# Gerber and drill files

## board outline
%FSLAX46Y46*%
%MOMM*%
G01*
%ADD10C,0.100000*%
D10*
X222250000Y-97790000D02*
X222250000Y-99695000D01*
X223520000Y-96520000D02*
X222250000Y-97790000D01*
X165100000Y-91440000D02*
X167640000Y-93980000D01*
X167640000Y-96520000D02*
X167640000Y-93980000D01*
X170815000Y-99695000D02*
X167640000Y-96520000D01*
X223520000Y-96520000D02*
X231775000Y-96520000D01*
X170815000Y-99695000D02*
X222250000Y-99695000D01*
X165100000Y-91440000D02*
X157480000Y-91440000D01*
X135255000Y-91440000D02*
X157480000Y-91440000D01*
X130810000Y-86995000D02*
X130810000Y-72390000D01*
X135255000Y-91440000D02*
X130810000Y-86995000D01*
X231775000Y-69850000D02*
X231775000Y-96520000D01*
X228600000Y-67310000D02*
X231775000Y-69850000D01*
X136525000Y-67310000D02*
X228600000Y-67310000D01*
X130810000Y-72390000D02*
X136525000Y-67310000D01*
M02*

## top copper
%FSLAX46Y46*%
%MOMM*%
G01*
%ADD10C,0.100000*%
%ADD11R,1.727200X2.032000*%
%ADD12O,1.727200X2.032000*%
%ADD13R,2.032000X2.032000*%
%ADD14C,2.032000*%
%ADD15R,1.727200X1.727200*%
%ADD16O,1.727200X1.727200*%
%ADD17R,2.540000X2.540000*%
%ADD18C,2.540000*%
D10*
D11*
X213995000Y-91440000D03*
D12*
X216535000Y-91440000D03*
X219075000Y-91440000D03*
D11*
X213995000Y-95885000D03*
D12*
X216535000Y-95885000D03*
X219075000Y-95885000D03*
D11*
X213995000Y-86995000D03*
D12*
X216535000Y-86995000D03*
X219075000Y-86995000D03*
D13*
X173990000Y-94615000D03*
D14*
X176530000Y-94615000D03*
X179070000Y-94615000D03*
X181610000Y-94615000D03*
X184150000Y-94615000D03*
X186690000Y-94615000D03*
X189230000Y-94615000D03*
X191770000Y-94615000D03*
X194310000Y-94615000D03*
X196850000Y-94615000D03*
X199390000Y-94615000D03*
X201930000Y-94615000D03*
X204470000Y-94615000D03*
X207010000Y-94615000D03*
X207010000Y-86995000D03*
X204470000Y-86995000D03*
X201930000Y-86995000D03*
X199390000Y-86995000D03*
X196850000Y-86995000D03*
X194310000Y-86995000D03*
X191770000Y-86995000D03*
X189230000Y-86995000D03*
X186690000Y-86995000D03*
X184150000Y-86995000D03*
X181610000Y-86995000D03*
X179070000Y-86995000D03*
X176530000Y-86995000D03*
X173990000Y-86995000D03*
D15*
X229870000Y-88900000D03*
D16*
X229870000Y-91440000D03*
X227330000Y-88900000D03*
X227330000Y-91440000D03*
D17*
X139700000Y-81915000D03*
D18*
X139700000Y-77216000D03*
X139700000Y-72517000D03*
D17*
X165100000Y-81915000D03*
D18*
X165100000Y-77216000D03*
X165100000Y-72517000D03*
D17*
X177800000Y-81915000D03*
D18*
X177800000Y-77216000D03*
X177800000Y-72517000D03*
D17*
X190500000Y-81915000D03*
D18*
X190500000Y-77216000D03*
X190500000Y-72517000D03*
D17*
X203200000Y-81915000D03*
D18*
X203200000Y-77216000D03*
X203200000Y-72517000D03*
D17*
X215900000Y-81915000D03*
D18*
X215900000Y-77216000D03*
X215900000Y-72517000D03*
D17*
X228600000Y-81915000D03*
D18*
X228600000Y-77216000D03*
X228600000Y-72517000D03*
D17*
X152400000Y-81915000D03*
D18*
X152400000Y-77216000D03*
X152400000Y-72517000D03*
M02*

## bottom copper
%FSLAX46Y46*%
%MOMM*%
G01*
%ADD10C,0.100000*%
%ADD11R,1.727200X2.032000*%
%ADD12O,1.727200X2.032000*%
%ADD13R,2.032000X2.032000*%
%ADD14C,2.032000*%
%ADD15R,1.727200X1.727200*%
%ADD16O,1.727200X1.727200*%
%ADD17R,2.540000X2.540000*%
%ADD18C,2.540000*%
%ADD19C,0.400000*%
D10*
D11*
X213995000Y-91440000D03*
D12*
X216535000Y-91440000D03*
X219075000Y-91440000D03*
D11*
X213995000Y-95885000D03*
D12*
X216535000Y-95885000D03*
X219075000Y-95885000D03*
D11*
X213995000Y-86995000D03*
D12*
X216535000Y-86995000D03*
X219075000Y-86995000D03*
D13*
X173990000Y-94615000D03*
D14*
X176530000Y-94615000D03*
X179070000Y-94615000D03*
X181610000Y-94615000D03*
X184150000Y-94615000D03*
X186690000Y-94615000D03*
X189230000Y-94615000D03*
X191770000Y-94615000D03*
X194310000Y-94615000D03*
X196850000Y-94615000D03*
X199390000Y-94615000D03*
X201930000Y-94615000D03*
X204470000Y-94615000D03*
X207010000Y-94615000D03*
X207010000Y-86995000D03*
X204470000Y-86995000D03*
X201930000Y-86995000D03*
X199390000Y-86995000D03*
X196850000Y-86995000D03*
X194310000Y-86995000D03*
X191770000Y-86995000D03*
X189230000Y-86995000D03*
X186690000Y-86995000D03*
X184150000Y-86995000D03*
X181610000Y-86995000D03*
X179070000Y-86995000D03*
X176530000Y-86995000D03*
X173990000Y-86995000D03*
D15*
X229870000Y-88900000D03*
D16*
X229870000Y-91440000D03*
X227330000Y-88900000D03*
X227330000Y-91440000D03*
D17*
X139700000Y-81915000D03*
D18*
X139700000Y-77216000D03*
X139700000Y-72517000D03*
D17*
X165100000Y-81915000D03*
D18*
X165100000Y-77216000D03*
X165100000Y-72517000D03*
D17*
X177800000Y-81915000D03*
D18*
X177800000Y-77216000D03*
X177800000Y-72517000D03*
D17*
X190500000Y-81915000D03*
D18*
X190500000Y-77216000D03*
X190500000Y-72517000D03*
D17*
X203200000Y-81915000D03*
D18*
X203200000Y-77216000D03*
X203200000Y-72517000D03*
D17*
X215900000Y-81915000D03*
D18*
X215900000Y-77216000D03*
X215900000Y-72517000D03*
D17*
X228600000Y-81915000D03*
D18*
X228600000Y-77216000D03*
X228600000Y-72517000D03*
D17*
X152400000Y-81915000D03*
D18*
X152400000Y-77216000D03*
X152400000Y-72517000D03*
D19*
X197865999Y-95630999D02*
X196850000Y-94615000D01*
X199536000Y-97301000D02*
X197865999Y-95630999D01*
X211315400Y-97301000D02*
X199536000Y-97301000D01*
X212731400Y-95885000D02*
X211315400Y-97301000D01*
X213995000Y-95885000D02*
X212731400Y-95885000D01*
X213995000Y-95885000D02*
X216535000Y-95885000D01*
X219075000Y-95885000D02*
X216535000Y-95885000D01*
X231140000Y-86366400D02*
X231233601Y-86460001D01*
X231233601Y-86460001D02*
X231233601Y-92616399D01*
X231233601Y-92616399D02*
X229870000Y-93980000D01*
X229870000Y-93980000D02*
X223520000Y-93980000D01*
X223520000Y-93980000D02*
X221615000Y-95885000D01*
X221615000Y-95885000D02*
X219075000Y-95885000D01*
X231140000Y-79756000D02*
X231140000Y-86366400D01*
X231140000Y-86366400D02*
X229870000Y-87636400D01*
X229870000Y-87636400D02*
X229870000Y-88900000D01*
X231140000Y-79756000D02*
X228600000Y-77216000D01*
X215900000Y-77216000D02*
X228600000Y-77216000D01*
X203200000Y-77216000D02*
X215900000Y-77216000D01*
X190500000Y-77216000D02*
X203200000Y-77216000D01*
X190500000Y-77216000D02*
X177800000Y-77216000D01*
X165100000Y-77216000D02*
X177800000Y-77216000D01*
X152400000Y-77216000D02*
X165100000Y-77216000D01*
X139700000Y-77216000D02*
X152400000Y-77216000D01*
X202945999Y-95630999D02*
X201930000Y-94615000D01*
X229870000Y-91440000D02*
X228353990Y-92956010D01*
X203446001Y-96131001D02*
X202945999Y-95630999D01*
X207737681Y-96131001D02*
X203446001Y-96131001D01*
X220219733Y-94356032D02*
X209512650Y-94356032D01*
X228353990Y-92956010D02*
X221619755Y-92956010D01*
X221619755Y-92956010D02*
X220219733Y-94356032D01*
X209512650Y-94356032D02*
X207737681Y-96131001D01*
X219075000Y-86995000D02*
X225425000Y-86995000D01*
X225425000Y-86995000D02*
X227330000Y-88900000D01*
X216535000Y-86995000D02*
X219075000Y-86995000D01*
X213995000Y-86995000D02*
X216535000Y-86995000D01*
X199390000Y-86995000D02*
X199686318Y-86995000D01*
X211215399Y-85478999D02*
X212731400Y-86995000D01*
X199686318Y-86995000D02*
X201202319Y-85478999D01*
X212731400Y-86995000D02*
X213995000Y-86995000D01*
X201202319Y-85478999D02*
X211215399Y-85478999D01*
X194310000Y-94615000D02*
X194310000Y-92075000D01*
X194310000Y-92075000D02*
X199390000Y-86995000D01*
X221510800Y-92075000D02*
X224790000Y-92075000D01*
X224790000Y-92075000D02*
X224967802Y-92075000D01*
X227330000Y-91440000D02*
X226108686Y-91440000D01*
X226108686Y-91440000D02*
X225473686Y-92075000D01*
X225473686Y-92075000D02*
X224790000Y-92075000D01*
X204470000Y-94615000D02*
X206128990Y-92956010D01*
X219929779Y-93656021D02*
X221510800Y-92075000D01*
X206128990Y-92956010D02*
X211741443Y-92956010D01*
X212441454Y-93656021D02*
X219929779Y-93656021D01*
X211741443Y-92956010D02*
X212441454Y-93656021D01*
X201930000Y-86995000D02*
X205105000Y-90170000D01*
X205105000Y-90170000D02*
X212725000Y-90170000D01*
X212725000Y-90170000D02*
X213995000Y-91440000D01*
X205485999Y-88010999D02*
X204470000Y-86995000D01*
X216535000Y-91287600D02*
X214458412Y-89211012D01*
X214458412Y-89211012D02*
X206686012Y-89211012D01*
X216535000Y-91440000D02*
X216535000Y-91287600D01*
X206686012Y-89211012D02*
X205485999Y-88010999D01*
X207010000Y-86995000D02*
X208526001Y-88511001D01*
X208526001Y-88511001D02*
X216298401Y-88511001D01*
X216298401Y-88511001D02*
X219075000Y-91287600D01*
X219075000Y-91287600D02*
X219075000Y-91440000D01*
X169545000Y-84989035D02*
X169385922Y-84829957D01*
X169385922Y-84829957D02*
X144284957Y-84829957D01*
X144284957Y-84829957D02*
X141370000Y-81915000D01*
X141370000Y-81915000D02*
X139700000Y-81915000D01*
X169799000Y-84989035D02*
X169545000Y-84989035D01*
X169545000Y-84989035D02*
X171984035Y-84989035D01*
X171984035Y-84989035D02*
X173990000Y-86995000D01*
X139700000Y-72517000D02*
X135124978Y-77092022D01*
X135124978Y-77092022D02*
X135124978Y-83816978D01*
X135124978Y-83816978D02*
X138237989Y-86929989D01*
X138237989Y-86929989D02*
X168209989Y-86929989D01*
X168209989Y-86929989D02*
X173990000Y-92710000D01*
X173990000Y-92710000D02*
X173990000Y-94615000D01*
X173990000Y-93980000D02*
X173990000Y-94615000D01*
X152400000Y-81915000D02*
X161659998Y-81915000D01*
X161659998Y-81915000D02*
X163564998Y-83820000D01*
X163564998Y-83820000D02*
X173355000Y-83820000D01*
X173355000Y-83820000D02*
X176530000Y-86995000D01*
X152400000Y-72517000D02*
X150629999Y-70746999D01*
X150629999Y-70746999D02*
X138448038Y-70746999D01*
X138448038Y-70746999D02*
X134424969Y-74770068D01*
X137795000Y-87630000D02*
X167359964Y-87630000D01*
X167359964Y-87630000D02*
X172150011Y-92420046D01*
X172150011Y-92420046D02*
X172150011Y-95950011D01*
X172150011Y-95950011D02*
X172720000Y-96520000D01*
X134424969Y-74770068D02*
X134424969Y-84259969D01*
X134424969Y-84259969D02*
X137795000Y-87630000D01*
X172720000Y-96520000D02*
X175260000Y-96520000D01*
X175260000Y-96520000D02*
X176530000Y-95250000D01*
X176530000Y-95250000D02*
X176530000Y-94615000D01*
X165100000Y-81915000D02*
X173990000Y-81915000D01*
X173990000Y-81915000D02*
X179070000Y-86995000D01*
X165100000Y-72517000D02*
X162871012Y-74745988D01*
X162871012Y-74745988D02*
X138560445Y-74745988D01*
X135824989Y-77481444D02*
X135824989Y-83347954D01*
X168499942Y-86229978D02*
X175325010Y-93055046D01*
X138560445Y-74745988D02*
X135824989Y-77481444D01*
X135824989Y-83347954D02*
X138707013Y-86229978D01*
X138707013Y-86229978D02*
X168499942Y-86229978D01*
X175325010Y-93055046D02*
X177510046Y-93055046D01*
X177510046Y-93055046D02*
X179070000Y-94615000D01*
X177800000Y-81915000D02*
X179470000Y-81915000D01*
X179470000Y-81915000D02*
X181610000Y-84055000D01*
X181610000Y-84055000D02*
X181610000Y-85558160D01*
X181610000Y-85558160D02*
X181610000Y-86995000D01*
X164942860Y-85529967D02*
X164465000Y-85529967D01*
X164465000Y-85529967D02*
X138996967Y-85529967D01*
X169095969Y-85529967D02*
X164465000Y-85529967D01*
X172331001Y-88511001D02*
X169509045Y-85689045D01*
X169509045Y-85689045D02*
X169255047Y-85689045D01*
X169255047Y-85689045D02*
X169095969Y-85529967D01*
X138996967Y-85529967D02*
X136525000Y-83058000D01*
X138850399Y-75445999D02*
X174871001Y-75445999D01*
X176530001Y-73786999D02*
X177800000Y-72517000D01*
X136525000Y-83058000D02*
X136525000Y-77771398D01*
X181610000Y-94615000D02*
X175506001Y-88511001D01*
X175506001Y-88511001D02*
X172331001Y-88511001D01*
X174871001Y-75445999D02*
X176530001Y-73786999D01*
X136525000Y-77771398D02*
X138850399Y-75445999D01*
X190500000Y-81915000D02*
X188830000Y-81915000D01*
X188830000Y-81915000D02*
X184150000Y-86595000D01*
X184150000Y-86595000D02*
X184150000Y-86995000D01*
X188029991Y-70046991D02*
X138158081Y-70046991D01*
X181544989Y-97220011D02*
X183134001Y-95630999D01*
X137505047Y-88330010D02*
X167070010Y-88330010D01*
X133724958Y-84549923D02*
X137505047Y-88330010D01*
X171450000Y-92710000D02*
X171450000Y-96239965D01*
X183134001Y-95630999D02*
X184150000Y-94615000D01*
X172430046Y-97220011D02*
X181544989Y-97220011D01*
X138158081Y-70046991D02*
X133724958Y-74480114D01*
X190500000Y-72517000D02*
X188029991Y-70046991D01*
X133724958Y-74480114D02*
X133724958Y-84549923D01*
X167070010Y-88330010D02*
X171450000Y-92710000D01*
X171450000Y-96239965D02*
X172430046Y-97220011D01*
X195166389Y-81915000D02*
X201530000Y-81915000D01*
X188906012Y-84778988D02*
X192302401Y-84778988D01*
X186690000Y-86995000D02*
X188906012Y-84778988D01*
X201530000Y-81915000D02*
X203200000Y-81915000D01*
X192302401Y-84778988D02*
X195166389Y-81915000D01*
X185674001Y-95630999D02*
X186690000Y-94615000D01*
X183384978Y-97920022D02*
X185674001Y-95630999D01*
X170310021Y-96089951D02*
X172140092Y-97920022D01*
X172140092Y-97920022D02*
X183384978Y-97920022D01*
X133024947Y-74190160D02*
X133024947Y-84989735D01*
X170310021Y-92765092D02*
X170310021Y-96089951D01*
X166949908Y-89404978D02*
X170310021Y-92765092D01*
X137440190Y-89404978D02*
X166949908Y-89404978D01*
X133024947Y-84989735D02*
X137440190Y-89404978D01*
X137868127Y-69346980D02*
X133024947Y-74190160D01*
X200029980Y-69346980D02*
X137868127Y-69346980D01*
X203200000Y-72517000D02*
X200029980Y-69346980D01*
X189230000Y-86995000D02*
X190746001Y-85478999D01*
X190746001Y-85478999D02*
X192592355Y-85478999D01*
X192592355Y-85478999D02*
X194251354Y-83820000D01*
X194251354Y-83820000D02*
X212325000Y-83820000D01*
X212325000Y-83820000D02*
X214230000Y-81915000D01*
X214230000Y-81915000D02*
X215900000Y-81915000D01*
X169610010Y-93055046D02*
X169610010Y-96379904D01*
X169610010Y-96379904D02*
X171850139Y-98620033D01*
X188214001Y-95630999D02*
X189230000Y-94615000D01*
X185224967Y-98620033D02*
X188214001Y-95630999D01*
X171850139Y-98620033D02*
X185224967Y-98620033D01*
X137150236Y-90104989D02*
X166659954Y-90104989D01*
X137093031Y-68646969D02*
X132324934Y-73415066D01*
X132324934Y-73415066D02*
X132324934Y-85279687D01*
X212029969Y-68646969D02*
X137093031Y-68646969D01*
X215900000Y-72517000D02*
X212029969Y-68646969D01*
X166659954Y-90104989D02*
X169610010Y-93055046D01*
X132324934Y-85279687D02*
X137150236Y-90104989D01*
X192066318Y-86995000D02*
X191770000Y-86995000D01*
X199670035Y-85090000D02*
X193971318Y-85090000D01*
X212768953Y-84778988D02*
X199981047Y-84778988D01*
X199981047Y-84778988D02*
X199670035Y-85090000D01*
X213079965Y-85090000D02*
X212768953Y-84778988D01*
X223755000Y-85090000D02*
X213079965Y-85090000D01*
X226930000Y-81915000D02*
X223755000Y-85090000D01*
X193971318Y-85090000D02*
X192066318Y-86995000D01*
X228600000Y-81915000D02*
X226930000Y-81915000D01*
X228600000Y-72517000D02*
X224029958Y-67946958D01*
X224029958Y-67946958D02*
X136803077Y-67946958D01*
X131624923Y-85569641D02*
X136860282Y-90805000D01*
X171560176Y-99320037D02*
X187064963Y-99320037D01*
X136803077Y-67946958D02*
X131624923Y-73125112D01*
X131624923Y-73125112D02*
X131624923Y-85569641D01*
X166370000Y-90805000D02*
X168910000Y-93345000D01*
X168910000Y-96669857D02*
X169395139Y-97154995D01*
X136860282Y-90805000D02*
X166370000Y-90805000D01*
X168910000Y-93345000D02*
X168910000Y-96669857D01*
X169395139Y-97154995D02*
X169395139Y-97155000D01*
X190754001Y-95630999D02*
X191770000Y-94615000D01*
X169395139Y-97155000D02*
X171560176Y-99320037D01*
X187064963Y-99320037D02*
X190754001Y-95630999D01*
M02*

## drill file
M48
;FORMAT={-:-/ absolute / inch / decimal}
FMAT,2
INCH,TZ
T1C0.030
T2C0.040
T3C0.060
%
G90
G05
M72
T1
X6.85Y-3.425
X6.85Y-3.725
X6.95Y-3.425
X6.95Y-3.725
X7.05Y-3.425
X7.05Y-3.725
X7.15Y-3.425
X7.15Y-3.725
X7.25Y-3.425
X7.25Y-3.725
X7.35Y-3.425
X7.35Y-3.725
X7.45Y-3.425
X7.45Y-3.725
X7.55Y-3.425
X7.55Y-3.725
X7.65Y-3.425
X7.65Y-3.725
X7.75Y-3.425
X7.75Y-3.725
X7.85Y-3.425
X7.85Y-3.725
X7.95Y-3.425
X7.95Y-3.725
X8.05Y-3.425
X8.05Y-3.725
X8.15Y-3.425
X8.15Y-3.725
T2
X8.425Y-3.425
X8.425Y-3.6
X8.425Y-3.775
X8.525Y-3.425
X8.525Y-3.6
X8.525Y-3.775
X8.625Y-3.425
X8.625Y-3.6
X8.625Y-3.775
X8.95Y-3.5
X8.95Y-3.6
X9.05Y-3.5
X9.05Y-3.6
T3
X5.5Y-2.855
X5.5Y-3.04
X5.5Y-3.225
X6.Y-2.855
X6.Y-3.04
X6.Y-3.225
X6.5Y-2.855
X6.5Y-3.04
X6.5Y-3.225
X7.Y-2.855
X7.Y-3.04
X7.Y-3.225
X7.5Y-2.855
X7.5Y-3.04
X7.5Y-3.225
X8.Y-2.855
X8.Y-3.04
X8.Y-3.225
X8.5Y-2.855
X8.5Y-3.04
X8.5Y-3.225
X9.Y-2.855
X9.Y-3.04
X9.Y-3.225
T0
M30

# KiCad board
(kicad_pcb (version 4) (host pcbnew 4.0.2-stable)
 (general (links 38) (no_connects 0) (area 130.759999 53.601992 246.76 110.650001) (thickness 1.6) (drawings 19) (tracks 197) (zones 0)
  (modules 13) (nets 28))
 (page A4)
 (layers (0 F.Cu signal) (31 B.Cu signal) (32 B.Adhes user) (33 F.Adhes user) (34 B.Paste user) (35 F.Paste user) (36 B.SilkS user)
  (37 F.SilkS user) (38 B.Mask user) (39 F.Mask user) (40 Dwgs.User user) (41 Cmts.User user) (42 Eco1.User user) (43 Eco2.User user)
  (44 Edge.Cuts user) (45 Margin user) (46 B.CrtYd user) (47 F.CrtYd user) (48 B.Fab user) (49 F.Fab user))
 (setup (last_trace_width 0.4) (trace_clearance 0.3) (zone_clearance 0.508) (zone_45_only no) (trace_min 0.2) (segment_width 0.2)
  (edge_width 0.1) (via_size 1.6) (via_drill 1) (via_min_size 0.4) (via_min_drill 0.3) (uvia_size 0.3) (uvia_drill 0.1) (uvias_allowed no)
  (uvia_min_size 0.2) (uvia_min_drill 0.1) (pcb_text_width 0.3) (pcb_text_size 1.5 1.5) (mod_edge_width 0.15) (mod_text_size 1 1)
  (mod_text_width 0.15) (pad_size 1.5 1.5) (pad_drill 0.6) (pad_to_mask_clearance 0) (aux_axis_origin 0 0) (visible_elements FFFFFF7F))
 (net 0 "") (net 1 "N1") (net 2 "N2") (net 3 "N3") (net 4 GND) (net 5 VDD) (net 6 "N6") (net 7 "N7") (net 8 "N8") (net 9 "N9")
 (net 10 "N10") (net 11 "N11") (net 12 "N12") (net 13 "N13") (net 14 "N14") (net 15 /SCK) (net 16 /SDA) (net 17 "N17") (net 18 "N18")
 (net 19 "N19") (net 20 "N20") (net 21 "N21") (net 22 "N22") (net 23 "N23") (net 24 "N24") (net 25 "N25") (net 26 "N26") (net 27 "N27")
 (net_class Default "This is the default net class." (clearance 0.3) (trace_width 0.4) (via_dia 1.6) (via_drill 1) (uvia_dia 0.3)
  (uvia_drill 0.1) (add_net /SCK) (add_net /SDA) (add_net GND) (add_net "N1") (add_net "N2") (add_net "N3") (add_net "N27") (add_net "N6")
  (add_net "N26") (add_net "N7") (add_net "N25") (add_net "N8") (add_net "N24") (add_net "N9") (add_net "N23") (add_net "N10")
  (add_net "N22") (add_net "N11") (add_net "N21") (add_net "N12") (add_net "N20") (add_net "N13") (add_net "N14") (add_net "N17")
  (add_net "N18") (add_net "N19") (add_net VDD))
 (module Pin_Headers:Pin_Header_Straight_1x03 (layer F.Cu) (at 213.995 91.44 90)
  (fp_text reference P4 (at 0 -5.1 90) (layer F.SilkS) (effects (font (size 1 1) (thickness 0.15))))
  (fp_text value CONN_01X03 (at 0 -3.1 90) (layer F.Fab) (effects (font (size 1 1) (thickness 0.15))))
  (pad 1 thru_hole rect (at 0 0 90) (size 2.032 1.7272) (drill 1.016) (layers *.Cu *.Mask F.SilkS) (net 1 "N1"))
  (pad 2 thru_hole oval (at 0 2.54 90) (size 2.032 1.7272) (drill 1.016) (layers *.Cu *.Mask F.SilkS) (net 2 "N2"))
  (pad 3 thru_hole oval (at 0 5.08 90) (size 2.032 1.7272) (drill 1.016) (layers *.Cu *.Mask F.SilkS) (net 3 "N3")))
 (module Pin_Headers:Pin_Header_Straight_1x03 (layer F.Cu) (at 213.995 95.885 90)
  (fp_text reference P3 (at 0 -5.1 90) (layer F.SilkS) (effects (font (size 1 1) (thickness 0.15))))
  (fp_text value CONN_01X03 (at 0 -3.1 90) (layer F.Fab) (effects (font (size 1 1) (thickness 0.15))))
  (pad 1 thru_hole rect (at 0 0 90) (size 2.032 1.7272) (drill 1.016) (layers *.Cu *.Mask F.SilkS) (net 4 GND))
  (pad 2 thru_hole oval (at 0 2.54 90) (size 2.032 1.7272) (drill 1.016) (layers *.Cu *.Mask F.SilkS) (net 4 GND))
  (pad 3 thru_hole oval (at 0 5.08 90) (size 2.032 1.7272) (drill 1.016) (layers *.Cu *.Mask F.SilkS) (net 4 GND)))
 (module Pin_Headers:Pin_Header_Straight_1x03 (layer F.Cu) (at 213.995 86.995 90)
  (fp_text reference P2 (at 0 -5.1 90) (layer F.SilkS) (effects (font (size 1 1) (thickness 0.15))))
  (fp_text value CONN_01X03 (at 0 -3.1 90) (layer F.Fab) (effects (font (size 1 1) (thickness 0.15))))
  (pad 1 thru_hole rect (at 0 0 90) (size 2.032 1.7272) (drill 1.016) (layers *.Cu *.Mask F.SilkS) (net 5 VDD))
  (pad 2 thru_hole oval (at 0 2.54 90) (size 2.032 1.7272) (drill 1.016) (layers *.Cu *.Mask F.SilkS) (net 5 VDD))
  (pad 3 thru_hole oval (at 0 5.08 90) (size 2.032 1.7272) (drill 1.016) (layers *.Cu *.Mask F.SilkS) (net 5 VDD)))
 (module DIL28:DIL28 (layer F.Cu) (at 173.99 94.615)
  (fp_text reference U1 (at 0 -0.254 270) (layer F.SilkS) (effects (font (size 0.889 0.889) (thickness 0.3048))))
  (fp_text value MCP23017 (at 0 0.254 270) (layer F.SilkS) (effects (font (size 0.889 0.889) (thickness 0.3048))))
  (pad 1 thru_hole rect (at 0 0) (size 2.032 2.032) (drill 0.762) (layers *.Cu *.Mask F.SilkS) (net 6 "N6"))
  (pad 2 thru_hole circle (at 2.54 0) (size 2.032 2.032) (drill 0.762) (layers *.Cu *.Mask F.SilkS) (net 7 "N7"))
  (pad 3 thru_hole circle (at 5.08 0) (size 2.032 2.032) (drill 0.762) (layers *.Cu *.Mask F.SilkS) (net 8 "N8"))
  (pad 4 thru_hole circle (at 7.62 0) (size 2.032 2.032) (drill 0.762) (layers *.Cu *.Mask F.SilkS) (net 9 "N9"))
  (pad 5 thru_hole circle (at 10.16 0) (size 2.032 2.032) (drill 0.762) (layers *.Cu *.Mask F.SilkS) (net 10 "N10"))
  (pad 6 thru_hole circle (at 12.7 0) (size 2.032 2.032) (drill 0.762) (layers *.Cu *.Mask F.SilkS) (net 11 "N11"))
  (pad 7 thru_hole circle (at 15.24 0) (size 2.032 2.032) (drill 0.762) (layers *.Cu *.Mask F.SilkS) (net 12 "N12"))
  (pad 8 thru_hole circle (at 17.78 0) (size 2.032 2.032) (drill 0.762) (layers *.Cu *.Mask F.SilkS) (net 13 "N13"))
  (pad 9 thru_hole circle (at 20.32 0) (size 2.032 2.032) (drill 0.762) (layers *.Cu *.Mask F.SilkS) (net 5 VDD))
  (pad 10 thru_hole circle (at 22.86 0) (size 2.032 2.032) (drill 0.762) (layers *.Cu *.Mask F.SilkS) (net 4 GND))
  (pad 11 thru_hole circle (at 25.4 0) (size 2.032 2.032) (drill 0.762) (layers *.Cu *.Mask F.SilkS) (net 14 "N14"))
  (pad 12 thru_hole circle (at 27.94 0) (size 2.032 2.032) (drill 0.762) (layers *.Cu *.Mask F.SilkS) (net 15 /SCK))
  (pad 13 thru_hole circle (at 30.48 0) (size 2.032 2.032) (drill 0.762) (layers *.Cu *.Mask F.SilkS) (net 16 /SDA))
  (pad 14 thru_hole circle (at 33.02 0) (size 2.032 2.032) (drill 0.762) (layers *.Cu *.Mask F.SilkS) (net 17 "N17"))
  (pad 15 thru_hole circle (at 33.02 -7.62 180) (size 2.032 2.032) (drill 0.762) (layers *.Cu *.Mask F.SilkS) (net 3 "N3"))
  (pad 16 thru_hole circle (at 30.48 -7.62 180) (size 2.032 2.032) (drill 0.762) (layers *.Cu *.Mask F.SilkS) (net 2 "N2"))
  (pad 17 thru_hole circle (at 27.94 -7.62 180) (size 2.032 2.032) (drill 0.762) (layers *.Cu *.Mask F.SilkS) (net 1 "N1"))
  (pad 18 thru_hole circle (at 25.4 -7.62 180) (size 2.032 2.032) (drill 0.762) (layers *.Cu *.Mask F.SilkS) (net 5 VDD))
  (pad 19 thru_hole circle (at 22.86 -7.62 180) (size 2.032 2.032) (drill 0.762) (layers *.Cu *.Mask F.SilkS) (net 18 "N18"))
  (pad 20 thru_hole circle (at 20.32 -7.62 180) (size 2.032 2.032) (drill 0.762) (layers *.Cu *.Mask F.SilkS) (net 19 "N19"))
  (pad 21 thru_hole circle (at 17.78 -7.62 180) (size 2.032 2.032) (drill 0.762) (layers *.Cu *.Mask F.SilkS) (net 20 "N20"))
  (pad 22 thru_hole circle (at 15.24 -7.62 180) (size 2.032 2.032) (drill 0.762) (layers *.Cu *.Mask F.SilkS) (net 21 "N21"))
  (pad 23 thru_hole circle (at 12.7 -7.62 180) (size 2.032 2.032) (drill 0.762) (layers *.Cu *.Mask F.SilkS) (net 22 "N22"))
  (pad 24 thru_hole circle (at 10.16 -7.62 180) (size 2.032 2.032) (drill 0.762) (layers *.Cu *.Mask F.SilkS) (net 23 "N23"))
  (pad 25 thru_hole circle (at 7.62 -7.62 180) (size 2.032 2.032) (drill 0.762) (layers *.Cu *.Mask F.SilkS) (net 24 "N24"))
  (pad 26 thru_hole circle (at 5.08 -7.62 180) (size 2.032 2.032) (drill 0.762) (layers *.Cu *.Mask F.SilkS) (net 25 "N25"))
  (pad 27 thru_hole circle (at 2.54 -7.62 180) (size 2.032 2.032) (drill 0.762) (layers *.Cu *.Mask F.SilkS) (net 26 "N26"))
  (pad 28 thru_hole circle (at 0 -7.62 180) (size 2.032 2.032) (drill 0.762) (layers *.Cu *.Mask F.SilkS) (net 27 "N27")))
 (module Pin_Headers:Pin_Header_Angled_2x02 (layer F.Cu) (at 229.87 88.9 270)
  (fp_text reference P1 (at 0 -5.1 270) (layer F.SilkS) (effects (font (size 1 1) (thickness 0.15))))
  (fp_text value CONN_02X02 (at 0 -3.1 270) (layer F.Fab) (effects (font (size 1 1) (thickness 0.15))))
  (pad 1 thru_hole rect (at 0 0 270) (size 1.7272 1.7272) (drill 1.016) (layers *.Cu *.Mask F.SilkS) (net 4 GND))
  (pad 2 thru_hole oval (at 2.54 0 270) (size 1.7272 1.7272) (drill 1.016) (layers *.Cu *.Mask F.SilkS) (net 15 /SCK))
  (pad 3 thru_hole oval (at 0 2.54 270) (size 1.7272 1.7272) (drill 1.016) (layers *.Cu *.Mask F.SilkS) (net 5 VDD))
  (pad 4 thru_hole oval (at 2.54 2.54 270) (size 1.7272 1.7272) (drill 1.016) (layers *.Cu *.Mask F.SilkS) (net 16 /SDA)))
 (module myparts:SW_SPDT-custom (layer F.Cu) (at 139.7 77.216 90)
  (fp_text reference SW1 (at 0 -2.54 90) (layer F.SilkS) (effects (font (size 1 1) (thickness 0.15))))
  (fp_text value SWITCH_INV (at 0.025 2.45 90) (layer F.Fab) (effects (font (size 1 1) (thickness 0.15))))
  (pad 1 thru_hole rect (at -4.699 0 90) (size 2.54 2.54) (drill 1.524) (layers *.Cu *.Mask F.SilkS) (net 27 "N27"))
  (pad 2 thru_hole circle (at 0 0 90) (size 2.54 2.54) (drill 1.524) (layers *.Cu *.Mask F.SilkS) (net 4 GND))
  (pad 3 thru_hole circle (at 4.699 0 90) (size 2.54 2.54) (drill 1.524) (layers *.Cu *.Mask F.SilkS) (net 6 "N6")))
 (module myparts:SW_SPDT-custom (layer F.Cu) (at 165.1 77.216 90)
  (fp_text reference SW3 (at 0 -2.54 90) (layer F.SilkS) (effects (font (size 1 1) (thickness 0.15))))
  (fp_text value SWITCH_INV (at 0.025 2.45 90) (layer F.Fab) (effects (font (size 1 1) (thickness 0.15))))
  (pad 1 thru_hole rect (at -4.699 0 90) (size 2.54 2.54) (drill 1.524) (layers *.Cu *.Mask F.SilkS) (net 25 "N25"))
  (pad 2 thru_hole circle (at 0 0 90) (size 2.54 2.54) (drill 1.524) (layers *.Cu *.Mask F.SilkS) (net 4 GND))
  (pad 3 thru_hole circle (at 4.699 0 90) (size 2.54 2.54) (drill 1.524) (layers *.Cu *.Mask F.SilkS) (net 8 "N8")))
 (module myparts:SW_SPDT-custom (layer F.Cu) (at 177.8 77.216 90)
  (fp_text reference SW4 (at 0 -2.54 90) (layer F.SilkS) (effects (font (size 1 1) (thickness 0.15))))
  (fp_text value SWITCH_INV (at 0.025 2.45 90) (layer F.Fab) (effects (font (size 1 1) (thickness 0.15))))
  (pad 1 thru_hole rect (at -4.699 0 90) (size 2.54 2.54) (drill 1.524) (layers *.Cu *.Mask F.SilkS) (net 24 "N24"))
  (pad 2 thru_hole circle (at 0 0 90) (size 2.54 2.54) (drill 1.524) (layers *.Cu *.Mask F.SilkS) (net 4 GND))
  (pad 3 thru_hole circle (at 4.699 0 90) (size 2.54 2.54) (drill 1.524) (layers *.Cu *.Mask F.SilkS) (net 9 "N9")))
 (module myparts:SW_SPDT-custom (layer F.Cu) (at 190.5 77.216 90)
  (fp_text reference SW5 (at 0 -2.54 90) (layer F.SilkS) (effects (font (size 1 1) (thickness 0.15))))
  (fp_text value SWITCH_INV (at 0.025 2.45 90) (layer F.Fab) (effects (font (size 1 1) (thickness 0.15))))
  (pad 1 thru_hole rect (at -4.699 0 90) (size 2.54 2.54) (drill 1.524) (layers *.Cu *.Mask F.SilkS) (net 23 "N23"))
  (pad 2 thru_hole circle (at 0 0 90) (size 2.54 2.54) (drill 1.524) (layers *.Cu *.Mask F.SilkS) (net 4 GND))
  (pad 3 thru_hole circle (at 4.699 0 90) (size 2.54 2.54) (drill 1.524) (layers *.Cu *.Mask F.SilkS) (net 10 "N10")))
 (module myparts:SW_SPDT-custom (layer F.Cu) (at 203.2 77.216 90)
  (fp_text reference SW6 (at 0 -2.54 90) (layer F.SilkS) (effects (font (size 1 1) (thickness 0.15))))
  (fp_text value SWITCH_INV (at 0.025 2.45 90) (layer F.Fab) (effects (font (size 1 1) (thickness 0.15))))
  (pad 1 thru_hole rect (at -4.699 0 90) (size 2.54 2.54) (drill 1.524) (layers *.Cu *.Mask F.SilkS) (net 22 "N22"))
  (pad 2 thru_hole circle (at 0 0 90) (size 2.54 2.54) (drill 1.524) (layers *.Cu *.Mask F.SilkS) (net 4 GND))
  (pad 3 thru_hole circle (at 4.699 0 90) (size 2.54 2.54) (drill 1.524) (layers *.Cu *.Mask F.SilkS) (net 11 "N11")))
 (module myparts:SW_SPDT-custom (layer F.Cu) (at 215.9 77.216 90)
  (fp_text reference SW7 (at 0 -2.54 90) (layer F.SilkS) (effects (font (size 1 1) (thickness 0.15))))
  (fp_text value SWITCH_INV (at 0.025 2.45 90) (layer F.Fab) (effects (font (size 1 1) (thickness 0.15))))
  (pad 1 thru_hole rect (at -4.699 0 90) (size 2.54 2.54) (drill 1.524) (layers *.Cu *.Mask F.SilkS) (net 21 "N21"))
  (pad 2 thru_hole circle (at 0 0 90) (size 2.54 2.54) (drill 1.524) (layers *.Cu *.Mask F.SilkS) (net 4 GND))
  (pad 3 thru_hole circle (at 4.699 0 90) (size 2.54 2.54) (drill 1.524) (layers *.Cu *.Mask F.SilkS) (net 12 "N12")))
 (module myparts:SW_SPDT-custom (layer F.Cu) (at 228.6 77.216 90)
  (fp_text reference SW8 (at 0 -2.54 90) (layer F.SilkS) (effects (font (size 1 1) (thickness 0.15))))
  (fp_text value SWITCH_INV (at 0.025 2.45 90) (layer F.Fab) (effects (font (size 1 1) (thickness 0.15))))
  (pad 1 thru_hole rect (at -4.699 0 90) (size 2.54 2.54) (drill 1.524) (layers *.Cu *.Mask F.SilkS) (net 20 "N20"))
  (pad 2 thru_hole circle (at 0 0 90) (size 2.54 2.54) (drill 1.524) (layers *.Cu *.Mask F.SilkS) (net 4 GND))
  (pad 3 thru_hole circle (at 4.699 0 90) (size 2.54 2.54) (drill 1.524) (layers *.Cu *.Mask F.SilkS) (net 13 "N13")))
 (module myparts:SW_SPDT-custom (layer F.Cu) (at 152.4 77.216 90)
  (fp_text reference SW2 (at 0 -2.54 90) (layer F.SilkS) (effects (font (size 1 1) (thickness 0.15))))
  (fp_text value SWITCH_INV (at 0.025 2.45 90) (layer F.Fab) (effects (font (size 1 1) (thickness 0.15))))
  (pad 1 thru_hole rect (at -4.699 0 90) (size 2.54 2.54) (drill 1.524) (layers *.Cu *.Mask F.SilkS) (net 26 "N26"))
  (pad 2 thru_hole circle (at 0 0 90) (size 2.54 2.54) (drill 1.524) (layers *.Cu *.Mask F.SilkS) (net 4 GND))
  (pad 3 thru_hole circle (at 4.699 0 90) (size 2.54 2.54) (drill 1.524) (layers *.Cu *.Mask F.SilkS) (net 7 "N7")))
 (gr_line (start 222.25 97.79) (end 222.25 99.695) (layer Edge.Cuts) (width 0.1))
 (gr_line (start 223.52 96.52) (end 222.25 97.79) (layer Edge.Cuts) (width 0.1))
 (gr_line (start 165.1 91.44) (end 167.64 93.98) (layer Edge.Cuts) (width 0.1))
 (gr_line (start 167.64 96.52) (end 167.64 93.98) (layer Edge.Cuts) (width 0.1))
 (gr_line (start 170.815 99.695) (end 167.64 96.52) (layer Edge.Cuts) (width 0.1))
 (gr_line (start 223.52 96.52) (end 231.775 96.52) (layer Edge.Cuts) (width 0.1))
 (gr_line (start 170.815 99.695) (end 222.25 99.695) (layer Edge.Cuts) (width 0.1))
 (gr_line (start 165.1 91.44) (end 157.48 91.44) (layer Edge.Cuts) (width 0.1))
 (gr_line (start 135.255 91.44) (end 157.48 91.44) (layer Edge.Cuts) (width 0.1))
 (gr_line (start 130.81 86.995) (end 130.81 72.39) (layer Edge.Cuts) (width 0.1))
 (gr_line (start 135.255 91.44) (end 130.81 86.995) (layer Edge.Cuts) (width 0.1))
 (gr_line (start 231.775 69.85) (end 231.775 96.52) (layer Edge.Cuts) (width 0.1))
 (gr_line (start 228.6 67.31) (end 231.775 69.85) (layer Edge.Cuts) (width 0.1))
 (gr_line (start 136.525 67.31) (end 228.6 67.31) (layer Edge.Cuts) (width 0.1))
 (gr_line (start 130.81 72.39) (end 136.525 67.31) (layer Edge.Cuts) (width 0.1))
 (segment (start 197.865999 95.630999) (end 196.85 94.615) (width 0.4) (layer B.Cu) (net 4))
 (segment (start 199.536 97.301) (end 197.865999 95.630999) (width 0.4) (layer B.Cu) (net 4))
 (segment (start 211.3154 97.301) (end 199.536 97.301) (width 0.4) (layer B.Cu) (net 4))
 (segment (start 212.7314 95.885) (end 211.3154 97.301) (width 0.4) (layer B.Cu) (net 4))
 (segment (start 213.995 95.885) (end 212.7314 95.885) (width 0.4) (layer B.Cu) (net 4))
 (segment (start 213.995 95.885) (end 216.535 95.885) (width 0.4) (layer B.Cu) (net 4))
 (segment (start 219.075 95.885) (end 216.535 95.885) (width 0.4) (layer B.Cu) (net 4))
 (segment (start 231.14 86.3664) (end 231.233601 86.460001) (width 0.4) (layer B.Cu) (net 4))
 (segment (start 231.233601 86.460001) (end 231.233601 92.616399) (width 0.4) (layer B.Cu) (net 4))
 (segment (start 231.233601 92.616399) (end 229.87 93.98) (width 0.4) (layer B.Cu) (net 4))
 (segment (start 229.87 93.98) (end 223.52 93.98) (width 0.4) (layer B.Cu) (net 4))
 (segment (start 223.52 93.98) (end 221.615 95.885) (width 0.4) (layer B.Cu) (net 4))
 (segment (start 221.615 95.885) (end 219.075 95.885) (width 0.4) (layer B.Cu) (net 4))
 (segment (start 231.14 79.756) (end 231.14 86.3664) (width 0.4) (layer B.Cu) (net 4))
 (segment (start 231.14 86.3664) (end 229.87 87.6364) (width 0.4) (layer B.Cu) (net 4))
 (segment (start 229.87 87.6364) (end 229.87 88.9) (width 0.4) (layer B.Cu) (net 4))
 (segment (start 231.14 79.756) (end 228.6 77.216) (width 0.4) (layer B.Cu) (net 4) (status 20))
 (segment (start 215.9 77.216) (end 228.6 77.216) (width 0.4) (layer B.Cu) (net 4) (status 30))
 (segment (start 203.2 77.216) (end 215.9 77.216) (width 0.4) (layer B.Cu) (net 4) (status 30))
 (segment (start 190.5 77.216) (end 203.2 77.216) (width 0.4) (layer B.Cu) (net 4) (status 30))
 (segment (start 190.5 77.216) (end 177.8 77.216) (width 0.4) (layer B.Cu) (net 4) (status 30))
 (segment (start 165.1 77.216) (end 177.8 77.216) (width 0.4) (layer B.Cu) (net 4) (status 30))
 (segment (start 152.4 77.216) (end 165.1 77.216) (width 0.4) (layer B.Cu) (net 4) (status 30))
 (segment (start 139.7 77.216) (end 152.4 77.216) (width 0.4) (layer B.Cu) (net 4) (status 30))
 (segment (start 202.945999 95.630999) (end 201.93 94.615) (width 0.4) (layer B.Cu) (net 15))
 (segment (start 229.87 91.44) (end 228.35399 92.95601) (width 0.4) (layer B.Cu) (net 15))
 (segment (start 203.446001 96.131001) (end 202.945999 95.630999) (width 0.4) (layer B.Cu) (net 15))
 (segment (start 207.737681 96.131001) (end 203.446001 96.131001) (width 0.4) (layer B.Cu) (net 15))
 (segment (start 220.219733 94.356032) (end 209.51265 94.356032) (width 0.4) (layer B.Cu) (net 15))
 (segment (start 228.35399 92.95601) (end 221.619755 92.95601) (width 0.4) (layer B.Cu) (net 15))
 (segment (start 221.619755 92.95601) (end 220.219733 94.356032) (width 0.4) (layer B.Cu) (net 15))
 (segment (start 209.51265 94.356032) (end 207.737681 96.131001) (width 0.4) (layer B.Cu) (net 15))
 (segment (start 219.075 86.995) (end 225.425 86.995) (width 0.4) (layer B.Cu) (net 5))
 (segment (start 225.425 86.995) (end 227.33 88.9) (width 0.4) (layer B.Cu) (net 5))
 (segment (start 216.535 86.995) (end 219.075 86.995) (width 0.4) (layer B.Cu) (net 5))
 (segment (start 213.995 86.995) (end 216.535 86.995) (width 0.4) (layer B.Cu) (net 5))
 (segment (start 199.39 86.995) (end 199.686318 86.995) (width 0.4) (layer B.Cu) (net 5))
 (segment (start 211.215399 85.478999) (end 212.7314 86.995) (width 0.4) (layer B.Cu) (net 5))
 (segment (start 199.686318 86.995) (end 201.202319 85.478999) (width 0.4) (layer B.Cu) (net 5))
 (segment (start 212.7314 86.995) (end 213.995 86.995) (width 0.4) (layer B.Cu) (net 5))
 (segment (start 201.202319 85.478999) (end 211.215399 85.478999) (width 0.4) (layer B.Cu) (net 5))
 (segment (start 194.31 94.615) (end 194.31 92.075) (width 0.4) (layer B.Cu) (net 5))
 (segment (start 194.31 92.075) (end 199.39 86.995) (width 0.4) (layer B.Cu) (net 5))
 (segment (start 221.5108 92.075) (end 224.79 92.075) (width 0.4) (layer B.Cu) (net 16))
 (segment (start 224.79 92.075) (end 224.967802 92.075) (width 0.4) (layer B.Cu) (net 16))
 (segment (start 227.33 91.44) (end 226.108686 91.44) (width 0.4) (layer B.Cu) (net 16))
 (segment (start 226.108686 91.44) (end 225.473686 92.075) (width 0.4) (layer B.Cu) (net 16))
 (segment (start 225.473686 92.075) (end 224.79 92.075) (width 0.4) (layer B.Cu) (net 16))
 (segment (start 204.47 94.615) (end 206.12899 92.95601) (width 0.4) (layer B.Cu) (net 16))
 (segment (start 219.929779 93.656021) (end 221.5108 92.075) (width 0.4) (layer B.Cu) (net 16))
 (segment (start 206.12899 92.95601) (end 211.741443 92.95601) (width 0.4) (layer B.Cu) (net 16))
 (segment (start 212.441454 93.656021) (end 219.929779 93.656021) (width 0.4) (layer B.Cu) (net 16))
 (segment (start 211.741443 92.95601) (end 212.441454 93.656021) (width 0.4) (layer B.Cu) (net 16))
 (segment (start 201.93 86.995) (end 205.105 90.17) (width 0.4) (layer B.Cu) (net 1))
 (segment (start 205.105 90.17) (end 212.725 90.17) (width 0.4) (layer B.Cu) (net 1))
 (segment (start 212.725 90.17) (end 213.995 91.44) (width 0.4) (layer B.Cu) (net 1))
 (segment (start 205.485999 88.010999) (end 204.47 86.995) (width 0.4) (layer B.Cu) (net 2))
 (segment (start 216.535 91.2876) (end 214.458412 89.211012) (width 0.4) (layer B.Cu) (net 2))
 (segment (start 214.458412 89.211012) (end 206.686012 89.211012) (width 0.4) (layer B.Cu) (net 2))
 (segment (start 216.535 91.44) (end 216.535 91.2876) (width 0.4) (layer B.Cu) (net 2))
 (segment (start 206.686012 89.211012) (end 205.485999 88.010999) (width 0.4) (layer B.Cu) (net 2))
 (segment (start 207.01 86.995) (end 208.526001 88.511001) (width 0.4) (layer B.Cu) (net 3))
 (segment (start 208.526001 88.511001) (end 216.298401 88.511001) (width 0.4) (layer B.Cu) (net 3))
 (segment (start 216.298401 88.511001) (end 219.075 91.2876) (width 0.4) (layer B.Cu) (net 3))
 (segment (start 219.075 91.2876) (end 219.075 91.44) (width 0.4) (layer B.Cu) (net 3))
 (segment (start 169.545 84.989035) (end 169.385922 84.829957) (width 0.4) (layer B.Cu) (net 27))
 (segment (start 169.385922 84.829957) (end 144.284957 84.829957) (width 0.4) (layer B.Cu) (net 27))
 (segment (start 144.284957 84.829957) (end 141.37 81.915) (width 0.4) (layer B.Cu) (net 27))
 (segment (start 141.37 81.915) (end 139.7 81.915) (width 0.4) (layer B.Cu) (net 27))
 (segment (start 169.799 84.989035) (end 169.545 84.989035) (width 0.4) (layer B.Cu) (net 27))
 (segment (start 169.545 84.989035) (end 171.984035 84.989035) (width 0.4) (layer B.Cu) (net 27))
 (segment (start 171.984035 84.989035) (end 173.99 86.995) (width 0.4) (layer B.Cu) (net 27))
 (segment (start 139.7 72.517) (end 135.124978 77.092022) (width 0.4) (layer B.Cu) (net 6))
 (segment (start 135.124978 77.092022) (end 135.124978 83.816978) (width 0.4) (layer B.Cu) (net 6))
 (segment (start 135.124978 83.816978) (end 138.237989 86.929989) (width 0.4) (layer B.Cu) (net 6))
 (segment (start 138.237989 86.929989) (end 168.209989 86.929989) (width 0.4) (layer B.Cu) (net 6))
 (segment (start 168.209989 86.929989) (end 173.99 92.71) (width 0.4) (layer B.Cu) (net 6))
 (segment (start 173.99 92.71) (end 173.99 94.615) (width 0.4) (layer B.Cu) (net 6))
 (segment (start 173.99 93.98) (end 173.99 94.615) (width 0.4) (layer B.Cu) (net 6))
 (segment (start 152.4 81.915) (end 161.659998 81.915) (width 0.4) (layer B.Cu) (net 26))
 (segment (start 161.659998 81.915) (end 163.564998 83.82) (width 0.4) (layer B.Cu) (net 26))
 (segment (start 163.564998 83.82) (end 173.355 83.82) (width 0.4) (layer B.Cu) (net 26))
 (segment (start 173.355 83.82) (end 176.53 86.995) (width 0.4) (layer B.Cu) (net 26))
 (segment (start 152.4 72.517) (end 150.629999 70.746999) (width 0.4) (layer B.Cu) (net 7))
 (segment (start 150.629999 70.746999) (end 138.448038 70.746999) (width 0.4) (layer B.Cu) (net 7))
 (segment (start 138.448038 70.746999) (end 134.424969 74.770068) (width 0.4) (layer B.Cu) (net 7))
 (segment (start 137.795 87.63) (end 167.359964 87.63) (width 0.4) (layer B.Cu) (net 7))
 (segment (start 167.359964 87.63) (end 172.150011 92.420046) (width 0.4) (layer B.Cu) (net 7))
 (segment (start 172.150011 92.420046) (end 172.150011 95.950011) (width 0.4) (layer B.Cu) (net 7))
 (segment (start 172.150011 95.950011) (end 172.72 96.52) (width 0.4) (layer B.Cu) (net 7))
 (segment (start 134.424969 74.770068) (end 134.424969 84.259969) (width 0.4) (layer B.Cu) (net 7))
 (segment (start 134.424969 84.259969) (end 137.795 87.63) (width 0.4) (layer B.Cu) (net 7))
 (segment (start 172.72 96.52) (end 175.26 96.52) (width 0.4) (layer B.Cu) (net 7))
 (segment (start 175.26 96.52) (end 176.53 95.25) (width 0.4) (layer B.Cu) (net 7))
 (segment (start 176.53 95.25) (end 176.53 94.615) (width 0.4) (layer B.Cu) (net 7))
 (segment (start 165.1 81.915) (end 173.99 81.915) (width 0.4) (layer B.Cu) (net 25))
 (segment (start 173.99 81.915) (end 179.07 86.995) (width 0.4) (layer B.Cu) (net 25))
 (segment (start 165.1 72.517) (end 162.871012 74.745988) (width 0.4) (layer B.Cu) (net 8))
 (segment (start 162.871012 74.745988) (end 138.560445 74.745988) (width 0.4) (layer B.Cu) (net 8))
 (segment (start 135.824989 77.481444) (end 135.824989 83.347954) (width 0.4) (layer B.Cu) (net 8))
 (segment (start 168.499942 86.229978) (end 175.32501 93.055046) (width 0.4) (layer B.Cu) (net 8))
 (segment (start 138.560445 74.745988) (end 135.824989 77.481444) (width 0.4) (layer B.Cu) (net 8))
 (segment (start 135.824989 83.347954) (end 138.707013 86.229978) (width 0.4) (layer B.Cu) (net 8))
 (segment (start 138.707013 86.229978) (end 168.499942 86.229978) (width 0.4) (layer B.Cu) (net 8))
 (segment (start 175.32501 93.055046) (end 177.510046 93.055046) (width 0.4) (layer B.Cu) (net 8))
 (segment (start 177.510046 93.055046) (end 179.07 94.615) (width 0.4) (layer B.Cu) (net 8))
 (segment (start 177.8 81.915) (end 179.47 81.915) (width 0.4) (layer B.Cu) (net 24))
 (segment (start 179.47 81.915) (end 181.61 84.055) (width 0.4) (layer B.Cu) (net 24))
 (segment (start 181.61 84.055) (end 181.61 85.55816) (width 0.4) (layer B.Cu) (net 24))
 (segment (start 181.61 85.55816) (end 181.61 86.995) (width 0.4) (layer B.Cu) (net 24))
 (segment (start 164.94286 85.529967) (end 164.465 85.529967) (width 0.4) (layer B.Cu) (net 9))
 (segment (start 164.465 85.529967) (end 138.996967 85.529967) (width 0.4) (layer B.Cu) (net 9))
 (segment (start 169.095969 85.529967) (end 164.465 85.529967) (width 0.4) (layer B.Cu) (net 9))
 (segment (start 172.331001 88.511001) (end 169.509045 85.689045) (width 0.4) (layer B.Cu) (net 9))
 (segment (start 169.509045 85.689045) (end 169.255047 85.689045) (width 0.4) (layer B.Cu) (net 9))
 (segment (start 169.255047 85.689045) (end 169.095969 85.529967) (width 0.4) (layer B.Cu) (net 9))
 (segment (start 138.996967 85.529967) (end 136.525 83.058) (width 0.4) (layer B.Cu) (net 9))
 (segment (start 138.850399 75.445999) (end 174.871001 75.445999) (width 0.4) (layer B.Cu) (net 9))
 (segment (start 176.530001 73.786999) (end 177.8 72.517) (width 0.4) (layer B.Cu) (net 9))
 (segment (start 136.525 83.058) (end 136.525 77.771398) (width 0.4) (layer B.Cu) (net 9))
 (segment (start 181.61 94.615) (end 175.506001 88.511001) (width 0.4) (layer B.Cu) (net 9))
 (segment (start 175.506001 88.511001) (end 172.331001 88.511001) (width 0.4) (layer B.Cu) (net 9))
 (segment (start 174.871001 75.445999) (end 176.530001 73.786999) (width 0.4) (layer B.Cu) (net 9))
 (segment (start 136.525 77.771398) (end 138.850399 75.445999) (width 0.4) (layer B.Cu) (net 9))
 (segment (start 190.5 81.915) (end 188.83 81.915) (width 0.4) (layer B.Cu) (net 23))
 (segment (start 188.83 81.915) (end 184.15 86.595) (width 0.4) (layer B.Cu) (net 23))
 (segment (start 184.15 86.595) (end 184.15 86.995) (width 0.4) (layer B.Cu) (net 23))
 (segment (start 188.029991 70.046991) (end 138.158081 70.046991) (width 0.4) (layer B.Cu) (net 10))
 (segment (start 181.544989 97.220011) (end 183.134001 95.630999) (width 0.4) (layer B.Cu) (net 10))
 (segment (start 137.505047 88.33001) (end 167.07001 88.33001) (width 0.4) (layer B.Cu) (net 10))
 (segment (start 133.724958 84.549923) (end 137.505047 88.33001) (width 0.4) (layer B.Cu) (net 10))
 (segment (start 171.45 92.71) (end 171.45 96.239965) (width 0.4) (layer B.Cu) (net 10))
 (segment (start 183.134001 95.630999) (end 184.15 94.615) (width 0.4) (layer B.Cu) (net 10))
 (segment (start 172.430046 97.220011) (end 181.544989 97.220011) (width 0.4) (layer B.Cu) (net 10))
 (segment (start 138.158081 70.046991) (end 133.724958 74.480114) (width 0.4) (layer B.Cu) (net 10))
 (segment (start 190.5 72.517) (end 188.029991 70.046991) (width 0.4) (layer B.Cu) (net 10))
 (segment (start 133.724958 74.480114) (end 133.724958 84.549923) (width 0.4) (layer B.Cu) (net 10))
 (segment (start 167.07001 88.33001) (end 171.45 92.71) (width 0.4) (layer B.Cu) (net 10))
 (segment (start 171.45 96.239965) (end 172.430046 97.220011) (width 0.4) (layer B.Cu) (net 10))
 (segment (start 195.166389 81.915) (end 201.53 81.915) (width 0.4) (layer B.Cu) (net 22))
 (segment (start 188.906012 84.778988) (end 192.302401 84.778988) (width 0.4) (layer B.Cu) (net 22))
 (segment (start 186.69 86.995) (end 188.906012 84.778988) (width 0.4) (layer B.Cu) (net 22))
 (segment (start 201.53 81.915) (end 203.2 81.915) (width 0.4) (layer B.Cu) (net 22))
 (segment (start 192.302401 84.778988) (end 195.166389 81.915) (width 0.4) (layer B.Cu) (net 22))
 (segment (start 185.674001 95.630999) (end 186.69 94.615) (width 0.4) (layer B.Cu) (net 11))
 (segment (start 183.384978 97.920022) (end 185.674001 95.630999) (width 0.4) (layer B.Cu) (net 11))
 (segment (start 170.310021 96.089951) (end 172.140092 97.920022) (width 0.4) (layer B.Cu) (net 11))
 (segment (start 172.140092 97.920022) (end 183.384978 97.920022) (width 0.4) (layer B.Cu) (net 11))
 (segment (start 133.024947 74.19016) (end 133.024947 84.989735) (width 0.4) (layer B.Cu) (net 11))
 (segment (start 170.310021 92.765092) (end 170.310021 96.089951) (width 0.4) (layer B.Cu) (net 11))
 (segment (start 166.949908 89.404978) (end 170.310021 92.765092) (width 0.4) (layer B.Cu) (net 11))
 (segment (start 137.44019 89.404978) (end 166.949908 89.404978) (width 0.4) (layer B.Cu) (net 11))
 (segment (start 133.024947 84.989735) (end 137.44019 89.404978) (width 0.4) (layer B.Cu) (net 11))
 (segment (start 137.868127 69.34698) (end 133.024947 74.19016) (width 0.4) (layer B.Cu) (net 11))
 (segment (start 200.02998 69.34698) (end 137.868127 69.34698) (width 0.4) (layer B.Cu) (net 11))
 (segment (start 203.2 72.517) (end 200.02998 69.34698) (width 0.4) (layer B.Cu) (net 11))
 (segment (start 189.23 86.995) (end 190.746001 85.478999) (width 0.4) (layer B.Cu) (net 21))
 (segment (start 190.746001 85.478999) (end 192.592355 85.478999) (width 0.4) (layer B.Cu) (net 21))
 (segment (start 192.592355 85.478999) (end 194.251354 83.82) (width 0.4) (layer B.Cu) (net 21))
 (segment (start 194.251354 83.82) (end 212.325 83.82) (width 0.4) (layer B.Cu) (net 21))
 (segment (start 212.325 83.82) (end 214.23 81.915) (width 0.4) (layer B.Cu) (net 21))
 (segment (start 214.23 81.915) (end 215.9 81.915) (width 0.4) (layer B.Cu) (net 21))
 (segment (start 169.61001 93.055046) (end 169.61001 96.379904) (width 0.4) (layer B.Cu) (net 12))
 (segment (start 169.61001 96.379904) (end 171.850139 98.620033) (width 0.4) (layer B.Cu) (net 12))
 (segment (start 188.214001 95.630999) (end 189.23 94.615) (width 0.4) (layer B.Cu) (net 12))
 (segment (start 185.224967 98.620033) (end 188.214001 95.630999) (width 0.4) (layer B.Cu) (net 12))
 (segment (start 171.850139 98.620033) (end 185.224967 98.620033) (width 0.4) (layer B.Cu) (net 12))
 (segment (start 137.150236 90.104989) (end 166.659954 90.104989) (width 0.4) (layer B.Cu) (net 12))
 (segment (start 137.093031 68.646969) (end 132.324934 73.415066) (width 0.4) (layer B.Cu) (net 12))
 (segment (start 132.324934 73.415066) (end 132.324934 85.279687) (width 0.4) (layer B.Cu) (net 12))
 (segment (start 212.029969 68.646969) (end 137.093031 68.646969) (width 0.4) (layer B.Cu) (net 12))
 (segment (start 215.9 72.517) (end 212.029969 68.646969) (width 0.4) (layer B.Cu) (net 12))
 (segment (start 166.659954 90.104989) (end 169.61001 93.055046) (width 0.4) (layer B.Cu) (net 12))
 (segment (start 132.324934 85.279687) (end 137.150236 90.104989) (width 0.4) (layer B.Cu) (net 12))
 (segment (start 192.066318 86.995) (end 191.77 86.995) (width 0.4) (layer B.Cu) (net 20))
 (segment (start 199.670035 85.09) (end 193.971318 85.09) (width 0.4) (layer B.Cu) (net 20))
 (segment (start 212.768953 84.778988) (end 199.981047 84.778988) (width 0.4) (layer B.Cu) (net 20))
 (segment (start 199.981047 84.778988) (end 199.670035 85.09) (width 0.4) (layer B.Cu) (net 20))
 (segment (start 213.079965 85.09) (end 212.768953 84.778988) (width 0.4) (layer B.Cu) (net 20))
 (segment (start 223.755 85.09) (end 213.079965 85.09) (width 0.4) (layer B.Cu) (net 20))
 (segment (start 226.93 81.915) (end 223.755 85.09) (width 0.4) (layer B.Cu) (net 20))
 (segment (start 193.971318 85.09) (end 192.066318 86.995) (width 0.4) (layer B.Cu) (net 20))
 (segment (start 228.6 81.915) (end 226.93 81.915) (width 0.4) (layer B.Cu) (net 20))
 (segment (start 228.6 72.517) (end 224.029958 67.946958) (width 0.4) (layer B.Cu) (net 13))
 (segment (start 224.029958 67.946958) (end 136.803077 67.946958) (width 0.4) (layer B.Cu) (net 13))
 (segment (start 131.624923 85.569641) (end 136.860282 90.805) (width 0.4) (layer B.Cu) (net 13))
 (segment (start 171.560176 99.320037) (end 187.064963 99.320037) (width 0.4) (layer B.Cu) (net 13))
 (segment (start 136.803077 67.946958) (end 131.624923 73.125112) (width 0.4) (layer B.Cu) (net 13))
 (segment (start 131.624923 73.125112) (end 131.624923 85.569641) (width 0.4) (layer B.Cu) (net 13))
 (segment (start 166.37 90.805) (end 168.91 93.345) (width 0.4) (layer B.Cu) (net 13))
 (segment (start 168.91 96.669857) (end 169.395139 97.154995) (width 0.4) (layer B.Cu) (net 13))
 (segment (start 136.860282 90.805) (end 166.37 90.805) (width 0.4) (layer B.Cu) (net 13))
 (segment (start 168.91 93.345) (end 168.91 96.669857) (width 0.4) (layer B.Cu) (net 13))
 (segment (start 169.395139 97.154995) (end 169.395139 97.155) (width 0.4) (layer B.Cu) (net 13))
 (segment (start 190.754001 95.630999) (end 191.77 94.615) (width 0.4) (layer B.Cu) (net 13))
 (segment (start 169.395139 97.155) (end 171.560176 99.320037) (width 0.4) (layer B.Cu) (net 13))
 (segment (start 187.064963 99.320037) (end 190.754001 95.630999) (width 0.4) (layer B.Cu) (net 13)))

